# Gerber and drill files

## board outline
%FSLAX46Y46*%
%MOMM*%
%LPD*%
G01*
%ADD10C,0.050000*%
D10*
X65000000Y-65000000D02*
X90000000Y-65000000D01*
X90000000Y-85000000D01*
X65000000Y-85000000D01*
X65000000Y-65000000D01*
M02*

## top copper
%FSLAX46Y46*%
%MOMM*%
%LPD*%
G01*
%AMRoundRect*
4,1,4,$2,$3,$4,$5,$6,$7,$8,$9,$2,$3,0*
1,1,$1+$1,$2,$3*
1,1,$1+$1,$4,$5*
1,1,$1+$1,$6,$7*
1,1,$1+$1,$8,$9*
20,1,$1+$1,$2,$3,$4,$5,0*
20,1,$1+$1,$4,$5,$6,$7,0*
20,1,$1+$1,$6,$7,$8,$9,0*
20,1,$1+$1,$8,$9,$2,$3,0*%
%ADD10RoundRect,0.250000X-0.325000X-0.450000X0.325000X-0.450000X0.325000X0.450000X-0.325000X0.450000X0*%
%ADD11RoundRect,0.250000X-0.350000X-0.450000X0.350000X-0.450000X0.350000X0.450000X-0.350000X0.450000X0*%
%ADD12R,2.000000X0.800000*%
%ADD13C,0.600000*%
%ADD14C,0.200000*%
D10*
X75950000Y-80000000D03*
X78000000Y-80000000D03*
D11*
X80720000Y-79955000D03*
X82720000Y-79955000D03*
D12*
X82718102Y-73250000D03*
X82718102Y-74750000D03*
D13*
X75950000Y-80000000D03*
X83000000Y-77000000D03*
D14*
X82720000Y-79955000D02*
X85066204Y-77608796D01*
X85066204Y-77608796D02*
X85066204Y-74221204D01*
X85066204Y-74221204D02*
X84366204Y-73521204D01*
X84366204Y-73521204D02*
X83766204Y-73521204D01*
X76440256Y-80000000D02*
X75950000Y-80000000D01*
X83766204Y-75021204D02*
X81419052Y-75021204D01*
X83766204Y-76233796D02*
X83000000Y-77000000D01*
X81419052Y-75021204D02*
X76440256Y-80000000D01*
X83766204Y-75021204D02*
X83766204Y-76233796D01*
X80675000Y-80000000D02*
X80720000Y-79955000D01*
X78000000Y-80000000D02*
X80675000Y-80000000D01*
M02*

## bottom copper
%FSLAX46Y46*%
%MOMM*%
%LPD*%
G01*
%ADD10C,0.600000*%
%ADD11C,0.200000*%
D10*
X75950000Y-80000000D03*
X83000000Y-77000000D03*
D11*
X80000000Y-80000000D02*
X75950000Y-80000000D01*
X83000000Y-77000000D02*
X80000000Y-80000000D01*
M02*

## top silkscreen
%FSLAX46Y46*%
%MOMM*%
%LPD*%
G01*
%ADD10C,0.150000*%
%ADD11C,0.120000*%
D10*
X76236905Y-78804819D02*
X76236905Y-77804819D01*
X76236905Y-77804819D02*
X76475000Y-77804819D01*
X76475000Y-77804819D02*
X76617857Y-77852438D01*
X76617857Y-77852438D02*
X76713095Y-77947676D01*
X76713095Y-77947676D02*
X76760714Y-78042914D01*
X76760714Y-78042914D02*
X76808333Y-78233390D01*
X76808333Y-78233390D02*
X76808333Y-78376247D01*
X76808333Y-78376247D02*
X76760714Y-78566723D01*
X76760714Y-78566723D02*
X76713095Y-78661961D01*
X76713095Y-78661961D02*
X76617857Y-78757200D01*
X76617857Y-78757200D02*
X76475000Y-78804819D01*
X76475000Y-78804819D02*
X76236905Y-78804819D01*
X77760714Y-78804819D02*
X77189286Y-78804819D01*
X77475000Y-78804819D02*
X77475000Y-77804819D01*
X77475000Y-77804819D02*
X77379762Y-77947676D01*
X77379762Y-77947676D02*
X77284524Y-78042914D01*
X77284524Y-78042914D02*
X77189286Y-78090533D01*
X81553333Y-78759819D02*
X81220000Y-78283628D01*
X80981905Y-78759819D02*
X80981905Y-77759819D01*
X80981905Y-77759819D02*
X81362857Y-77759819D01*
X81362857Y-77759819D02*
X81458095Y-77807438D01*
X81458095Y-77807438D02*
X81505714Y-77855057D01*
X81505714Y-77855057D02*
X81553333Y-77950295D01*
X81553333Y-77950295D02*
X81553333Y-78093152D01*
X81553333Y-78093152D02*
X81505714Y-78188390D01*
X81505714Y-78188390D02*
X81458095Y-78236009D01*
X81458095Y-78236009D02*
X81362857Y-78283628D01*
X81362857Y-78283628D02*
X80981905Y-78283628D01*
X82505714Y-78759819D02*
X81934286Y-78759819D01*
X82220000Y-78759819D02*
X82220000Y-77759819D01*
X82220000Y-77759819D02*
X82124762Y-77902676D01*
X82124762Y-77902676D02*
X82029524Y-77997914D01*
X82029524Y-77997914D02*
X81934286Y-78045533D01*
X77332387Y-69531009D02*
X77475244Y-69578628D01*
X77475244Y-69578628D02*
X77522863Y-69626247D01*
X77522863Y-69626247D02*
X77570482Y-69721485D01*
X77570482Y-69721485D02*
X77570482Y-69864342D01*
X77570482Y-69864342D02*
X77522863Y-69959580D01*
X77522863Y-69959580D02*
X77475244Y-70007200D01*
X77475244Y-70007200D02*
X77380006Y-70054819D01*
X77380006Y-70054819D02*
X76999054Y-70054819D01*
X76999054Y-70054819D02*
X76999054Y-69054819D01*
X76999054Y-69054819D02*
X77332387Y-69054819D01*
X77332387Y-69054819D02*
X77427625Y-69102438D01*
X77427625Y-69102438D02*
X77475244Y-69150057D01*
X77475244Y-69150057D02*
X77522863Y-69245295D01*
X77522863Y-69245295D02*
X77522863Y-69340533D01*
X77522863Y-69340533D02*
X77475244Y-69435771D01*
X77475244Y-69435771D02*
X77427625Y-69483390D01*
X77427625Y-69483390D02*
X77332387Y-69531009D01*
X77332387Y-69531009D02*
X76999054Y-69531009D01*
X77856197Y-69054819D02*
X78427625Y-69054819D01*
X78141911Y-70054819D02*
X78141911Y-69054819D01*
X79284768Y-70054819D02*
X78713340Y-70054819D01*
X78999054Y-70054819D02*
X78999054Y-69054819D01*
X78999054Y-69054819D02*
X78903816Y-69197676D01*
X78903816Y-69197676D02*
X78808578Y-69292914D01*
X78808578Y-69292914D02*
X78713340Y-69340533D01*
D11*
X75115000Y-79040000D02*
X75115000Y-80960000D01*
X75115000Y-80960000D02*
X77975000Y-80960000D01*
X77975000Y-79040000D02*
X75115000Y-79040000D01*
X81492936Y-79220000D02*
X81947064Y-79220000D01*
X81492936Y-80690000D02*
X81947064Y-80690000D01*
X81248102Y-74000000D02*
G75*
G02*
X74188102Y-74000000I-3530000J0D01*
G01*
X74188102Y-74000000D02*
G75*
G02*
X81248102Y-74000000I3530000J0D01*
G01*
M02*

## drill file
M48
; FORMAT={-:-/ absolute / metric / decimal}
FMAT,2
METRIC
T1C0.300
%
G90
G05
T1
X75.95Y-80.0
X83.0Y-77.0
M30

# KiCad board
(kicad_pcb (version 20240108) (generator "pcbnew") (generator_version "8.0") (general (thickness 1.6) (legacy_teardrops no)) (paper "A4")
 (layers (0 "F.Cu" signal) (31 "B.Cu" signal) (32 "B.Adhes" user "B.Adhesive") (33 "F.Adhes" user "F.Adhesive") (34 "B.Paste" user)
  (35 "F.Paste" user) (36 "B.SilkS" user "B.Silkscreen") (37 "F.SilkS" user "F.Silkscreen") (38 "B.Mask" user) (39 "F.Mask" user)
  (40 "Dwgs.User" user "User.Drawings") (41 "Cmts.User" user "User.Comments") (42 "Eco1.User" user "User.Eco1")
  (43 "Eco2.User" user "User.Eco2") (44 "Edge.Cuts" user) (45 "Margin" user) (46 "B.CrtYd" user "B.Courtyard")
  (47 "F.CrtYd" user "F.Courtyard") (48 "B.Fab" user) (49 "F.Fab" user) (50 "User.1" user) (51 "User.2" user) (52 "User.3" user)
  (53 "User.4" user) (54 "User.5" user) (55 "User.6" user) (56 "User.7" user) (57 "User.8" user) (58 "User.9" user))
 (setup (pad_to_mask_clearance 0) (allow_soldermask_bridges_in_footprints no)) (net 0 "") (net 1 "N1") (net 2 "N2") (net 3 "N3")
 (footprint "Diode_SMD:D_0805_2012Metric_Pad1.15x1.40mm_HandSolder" (layer "F.Cu") (at 76.975 80)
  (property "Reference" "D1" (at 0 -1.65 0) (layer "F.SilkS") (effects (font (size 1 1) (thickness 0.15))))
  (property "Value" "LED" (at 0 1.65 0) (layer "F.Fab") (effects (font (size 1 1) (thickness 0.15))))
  (fp_line (start -1.86 -0.96) (end -1.86 0.96) (stroke (width 0.12) (type solid)) (layer "F.SilkS"))
  (fp_line (start -1.86 0.96) (end 1 0.96) (stroke (width 0.12) (type solid)) (layer "F.SilkS"))
  (fp_line (start 1 -0.96) (end -1.86 -0.96) (stroke (width 0.12) (type solid)) (layer "F.SilkS"))
  (pad "1" smd roundrect (at -1.025 0) (size 1.15 1.4) (layers "F.Cu" "F.Paste" "F.Mask") (roundrect_rratio 0.217391) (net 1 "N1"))
  (pad "2" smd roundrect (at 1.025 0) (size 1.15 1.4) (layers "F.Cu" "F.Paste" "F.Mask") (roundrect_rratio 0.217391) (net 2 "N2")))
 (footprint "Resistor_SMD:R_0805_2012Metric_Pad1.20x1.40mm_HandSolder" (layer "F.Cu") (at 81.72 79.955)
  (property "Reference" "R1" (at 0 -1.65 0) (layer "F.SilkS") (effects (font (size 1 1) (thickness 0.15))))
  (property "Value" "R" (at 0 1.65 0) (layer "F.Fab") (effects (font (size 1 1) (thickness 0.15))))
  (fp_line (start -0.227064 -0.735) (end 0.227064 -0.735) (stroke (width 0.12) (type solid)) (layer "F.SilkS"))
  (fp_line (start -0.227064 0.735) (end 0.227064 0.735) (stroke (width 0.12) (type solid)) (layer "F.SilkS"))
  (pad "1" smd roundrect (at -1 0) (size 1.2 1.4) (layers "F.Cu" "F.Paste" "F.Mask") (roundrect_rratio 0.208333) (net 2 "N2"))
  (pad "2" smd roundrect (at 1 0) (size 1.2 1.4) (layers "F.Cu" "F.Paste" "F.Mask") (roundrect_rratio 0.208333) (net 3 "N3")))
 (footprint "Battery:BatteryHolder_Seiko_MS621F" (layer "F.Cu") (at 82.718102 74)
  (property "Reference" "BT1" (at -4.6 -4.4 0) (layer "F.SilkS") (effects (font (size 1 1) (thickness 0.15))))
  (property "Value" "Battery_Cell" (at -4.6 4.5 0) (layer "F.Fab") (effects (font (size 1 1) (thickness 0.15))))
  (fp_circle (center -5 0) (end -1.47 0) (stroke (width 0.12) (type solid)) (fill none) (layer "F.SilkS"))
  (pad "1" smd rect (at 0 -0.75) (size 2 0.8) (layers "F.Cu" "F.Paste" "F.Mask") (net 3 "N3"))
  (pad "2" smd rect (at 0 0.75) (size 2 0.8) (layers "F.Cu" "F.Paste" "F.Mask") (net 1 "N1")))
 (gr_rect (start 65 65) (end 90 85) (stroke (width 0.05) (type default)) (fill none) (layer "Edge.Cuts"))
 (segment (start 82.72 79.955) (end 85.066204 77.608796) (width 0.2) (layer "F.Cu") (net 3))
 (segment (start 85.066204 77.608796) (end 85.066204 74.221204) (width 0.2) (layer "F.Cu") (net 3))
 (segment (start 85.066204 74.221204) (end 84.366204 73.521204) (width 0.2) (layer "F.Cu") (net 3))
 (segment (start 84.366204 73.521204) (end 83.766204 73.521204) (width 0.2) (layer "F.Cu") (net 3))
 (segment (start 76.440256 80) (end 75.95 80) (width 0.2) (layer "F.Cu") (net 1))
 (segment (start 83.766204 75.021204) (end 81.419052 75.021204) (width 0.2) (layer "F.Cu") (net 1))
 (segment (start 83.766204 76.233796) (end 83 77) (width 0.2) (layer "F.Cu") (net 1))
 (segment (start 81.419052 75.021204) (end 76.440256 80) (width 0.2) (layer "F.Cu") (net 1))
 (segment (start 83.766204 75.021204) (end 83.766204 76.233796) (width 0.2) (layer "F.Cu") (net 1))
 (via (at 75.95 80) (size 0.6) (drill 0.3) (layers "F.Cu" "B.Cu") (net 1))
 (via (at 83 77) (size 0.6) (drill 0.3) (layers "F.Cu" "B.Cu") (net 1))
 (segment (start 80 80) (end 75.95 80) (width 0.2) (layer "B.Cu") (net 1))
 (segment (start 83 77) (end 80 80) (width 0.2) (layer "B.Cu") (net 1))
 (segment (start 80.675 80) (end 80.72 79.955) (width 0.2) (layer "F.Cu") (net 2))
 (segment (start 78 80) (end 80.675 80) (width 0.2) (layer "F.Cu") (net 2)))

